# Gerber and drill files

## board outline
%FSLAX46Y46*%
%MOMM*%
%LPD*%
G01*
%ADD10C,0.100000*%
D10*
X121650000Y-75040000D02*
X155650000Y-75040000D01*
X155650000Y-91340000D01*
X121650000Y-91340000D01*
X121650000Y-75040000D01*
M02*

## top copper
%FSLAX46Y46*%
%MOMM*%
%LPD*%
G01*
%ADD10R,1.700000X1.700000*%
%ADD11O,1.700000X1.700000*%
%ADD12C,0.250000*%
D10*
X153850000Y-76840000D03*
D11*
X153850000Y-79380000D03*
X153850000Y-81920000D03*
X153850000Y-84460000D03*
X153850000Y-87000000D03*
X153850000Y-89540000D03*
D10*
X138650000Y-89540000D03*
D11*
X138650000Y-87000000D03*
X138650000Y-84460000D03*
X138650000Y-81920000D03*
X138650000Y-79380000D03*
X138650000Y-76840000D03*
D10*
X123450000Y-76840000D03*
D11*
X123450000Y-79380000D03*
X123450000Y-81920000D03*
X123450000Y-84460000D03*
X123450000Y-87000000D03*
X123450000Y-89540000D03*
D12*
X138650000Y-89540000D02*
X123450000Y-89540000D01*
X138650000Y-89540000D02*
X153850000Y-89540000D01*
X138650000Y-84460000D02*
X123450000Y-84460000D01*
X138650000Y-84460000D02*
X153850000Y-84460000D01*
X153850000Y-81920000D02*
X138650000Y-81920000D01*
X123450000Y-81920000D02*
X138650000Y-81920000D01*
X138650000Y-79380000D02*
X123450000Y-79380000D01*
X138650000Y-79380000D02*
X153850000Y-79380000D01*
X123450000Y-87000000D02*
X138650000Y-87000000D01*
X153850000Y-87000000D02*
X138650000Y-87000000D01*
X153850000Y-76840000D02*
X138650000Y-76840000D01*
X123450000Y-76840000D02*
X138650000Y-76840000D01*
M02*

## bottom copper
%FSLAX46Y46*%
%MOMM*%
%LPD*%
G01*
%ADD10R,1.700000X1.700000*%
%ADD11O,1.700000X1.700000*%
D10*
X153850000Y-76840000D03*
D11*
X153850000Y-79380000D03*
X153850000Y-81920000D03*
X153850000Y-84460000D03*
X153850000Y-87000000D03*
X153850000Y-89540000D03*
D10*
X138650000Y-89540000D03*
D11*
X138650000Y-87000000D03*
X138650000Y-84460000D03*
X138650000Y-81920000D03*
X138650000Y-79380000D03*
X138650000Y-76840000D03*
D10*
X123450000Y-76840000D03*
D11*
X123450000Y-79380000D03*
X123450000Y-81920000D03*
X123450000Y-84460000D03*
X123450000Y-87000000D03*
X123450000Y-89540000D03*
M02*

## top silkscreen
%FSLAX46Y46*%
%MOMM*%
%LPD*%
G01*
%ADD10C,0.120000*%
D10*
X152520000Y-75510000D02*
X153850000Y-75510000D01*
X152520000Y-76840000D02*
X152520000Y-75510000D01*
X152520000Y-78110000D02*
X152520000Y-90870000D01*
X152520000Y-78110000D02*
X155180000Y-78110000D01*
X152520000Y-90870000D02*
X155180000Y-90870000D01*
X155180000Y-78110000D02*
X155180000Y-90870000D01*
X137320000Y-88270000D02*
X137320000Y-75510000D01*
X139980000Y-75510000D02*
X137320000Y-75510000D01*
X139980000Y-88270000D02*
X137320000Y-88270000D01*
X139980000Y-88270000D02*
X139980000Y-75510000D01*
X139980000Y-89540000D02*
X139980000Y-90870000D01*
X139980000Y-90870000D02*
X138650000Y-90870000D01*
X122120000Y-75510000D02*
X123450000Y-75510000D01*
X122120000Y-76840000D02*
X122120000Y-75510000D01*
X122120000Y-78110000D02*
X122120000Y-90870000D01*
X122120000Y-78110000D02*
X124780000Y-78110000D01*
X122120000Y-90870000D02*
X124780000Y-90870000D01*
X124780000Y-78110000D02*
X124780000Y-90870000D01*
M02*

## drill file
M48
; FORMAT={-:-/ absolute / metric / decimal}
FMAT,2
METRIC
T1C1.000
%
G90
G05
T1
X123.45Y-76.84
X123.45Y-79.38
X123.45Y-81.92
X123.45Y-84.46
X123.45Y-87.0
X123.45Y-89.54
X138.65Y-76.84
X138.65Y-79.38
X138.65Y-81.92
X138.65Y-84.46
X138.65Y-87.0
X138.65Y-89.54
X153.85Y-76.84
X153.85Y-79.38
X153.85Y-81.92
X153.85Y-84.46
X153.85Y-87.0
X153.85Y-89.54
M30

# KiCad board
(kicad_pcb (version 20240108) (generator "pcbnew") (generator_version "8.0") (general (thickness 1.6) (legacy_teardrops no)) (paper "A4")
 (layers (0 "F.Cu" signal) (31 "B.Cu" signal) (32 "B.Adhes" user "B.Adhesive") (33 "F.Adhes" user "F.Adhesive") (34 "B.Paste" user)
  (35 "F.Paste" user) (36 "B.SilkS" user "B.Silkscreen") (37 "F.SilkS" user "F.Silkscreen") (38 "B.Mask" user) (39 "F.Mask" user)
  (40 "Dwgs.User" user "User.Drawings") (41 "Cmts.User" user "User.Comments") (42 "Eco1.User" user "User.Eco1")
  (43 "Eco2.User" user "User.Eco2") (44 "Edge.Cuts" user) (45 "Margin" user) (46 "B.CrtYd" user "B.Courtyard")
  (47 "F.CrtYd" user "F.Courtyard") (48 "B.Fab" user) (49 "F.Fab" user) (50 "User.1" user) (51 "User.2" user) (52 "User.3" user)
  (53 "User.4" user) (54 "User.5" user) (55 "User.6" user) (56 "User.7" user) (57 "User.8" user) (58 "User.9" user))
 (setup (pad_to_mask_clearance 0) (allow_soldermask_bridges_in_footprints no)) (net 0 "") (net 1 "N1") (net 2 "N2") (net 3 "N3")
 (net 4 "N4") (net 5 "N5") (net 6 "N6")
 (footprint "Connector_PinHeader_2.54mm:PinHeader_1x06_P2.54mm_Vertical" (layer "F.Cu") (at 153.85 76.84)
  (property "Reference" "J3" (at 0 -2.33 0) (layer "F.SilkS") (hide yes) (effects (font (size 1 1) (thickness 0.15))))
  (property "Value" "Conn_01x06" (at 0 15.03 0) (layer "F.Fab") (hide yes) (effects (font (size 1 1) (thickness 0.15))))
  (fp_line (start -1.33 -1.33) (end 0 -1.33) (stroke (width 0.12) (type solid)) (layer "F.SilkS"))
  (fp_line (start -1.33 0) (end -1.33 -1.33) (stroke (width 0.12) (type solid)) (layer "F.SilkS"))
  (fp_line (start -1.33 1.27) (end -1.33 14.03) (stroke (width 0.12) (type solid)) (layer "F.SilkS"))
  (fp_line (start -1.33 1.27) (end 1.33 1.27) (stroke (width 0.12) (type solid)) (layer "F.SilkS"))
  (fp_line (start -1.33 14.03) (end 1.33 14.03) (stroke (width 0.12) (type solid)) (layer "F.SilkS"))
  (fp_line (start 1.33 1.27) (end 1.33 14.03) (stroke (width 0.12) (type solid)) (layer "F.SilkS"))
  (pad "1" thru_hole rect (at 0 0) (size 1.7 1.7) (drill 1) (layers "*.Cu" "*.Mask") (remove_unused_layers no) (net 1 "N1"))
  (pad "2" thru_hole oval (at 0 2.54) (size 1.7 1.7) (drill 1) (layers "*.Cu" "*.Mask") (remove_unused_layers no) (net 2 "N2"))
  (pad "3" thru_hole oval (at 0 5.08) (size 1.7 1.7) (drill 1) (layers "*.Cu" "*.Mask") (remove_unused_layers no) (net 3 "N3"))
  (pad "4" thru_hole oval (at 0 7.62) (size 1.7 1.7) (drill 1) (layers "*.Cu" "*.Mask") (remove_unused_layers no) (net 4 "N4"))
  (pad "5" thru_hole oval (at 0 10.16) (size 1.7 1.7) (drill 1) (layers "*.Cu" "*.Mask") (remove_unused_layers no) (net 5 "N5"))
  (pad "6" thru_hole oval (at 0 12.7) (size 1.7 1.7) (drill 1) (layers "*.Cu" "*.Mask") (remove_unused_layers no) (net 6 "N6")))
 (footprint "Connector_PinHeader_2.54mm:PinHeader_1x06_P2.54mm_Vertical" (layer "F.Cu") (at 138.65 89.54 180)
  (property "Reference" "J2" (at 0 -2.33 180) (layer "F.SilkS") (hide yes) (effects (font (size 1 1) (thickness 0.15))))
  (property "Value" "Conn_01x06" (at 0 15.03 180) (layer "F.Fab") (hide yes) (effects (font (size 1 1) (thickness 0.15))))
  (fp_line (start 1.33 1.27) (end 1.33 14.03) (stroke (width 0.12) (type solid)) (layer "F.SilkS"))
  (fp_line (start -1.33 14.03) (end 1.33 14.03) (stroke (width 0.12) (type solid)) (layer "F.SilkS"))
  (fp_line (start -1.33 1.27) (end 1.33 1.27) (stroke (width 0.12) (type solid)) (layer "F.SilkS"))
  (fp_line (start -1.33 1.27) (end -1.33 14.03) (stroke (width 0.12) (type solid)) (layer "F.SilkS"))
  (fp_line (start -1.33 0) (end -1.33 -1.33) (stroke (width 0.12) (type solid)) (layer "F.SilkS"))
  (fp_line (start -1.33 -1.33) (end 0 -1.33) (stroke (width 0.12) (type solid)) (layer "F.SilkS"))
  (pad "1" thru_hole rect (at 0 0 180) (size 1.7 1.7) (drill 1) (layers "*.Cu" "*.Mask") (remove_unused_layers no) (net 6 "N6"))
  (pad "2" thru_hole oval (at 0 2.54 180) (size 1.7 1.7) (drill 1) (layers "*.Cu" "*.Mask") (remove_unused_layers no) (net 5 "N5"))
  (pad "3" thru_hole oval (at 0 5.08 180) (size 1.7 1.7) (drill 1) (layers "*.Cu" "*.Mask") (remove_unused_layers no) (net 4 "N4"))
  (pad "4" thru_hole oval (at 0 7.62 180) (size 1.7 1.7) (drill 1) (layers "*.Cu" "*.Mask") (remove_unused_layers no) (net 3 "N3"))
  (pad "5" thru_hole oval (at 0 10.16 180) (size 1.7 1.7) (drill 1) (layers "*.Cu" "*.Mask") (remove_unused_layers no) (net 2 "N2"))
  (pad "6" thru_hole oval (at 0 12.7 180) (size 1.7 1.7) (drill 1) (layers "*.Cu" "*.Mask") (remove_unused_layers no) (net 1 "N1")))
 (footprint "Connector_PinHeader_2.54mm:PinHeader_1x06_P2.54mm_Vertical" (layer "F.Cu") (at 123.45 76.84)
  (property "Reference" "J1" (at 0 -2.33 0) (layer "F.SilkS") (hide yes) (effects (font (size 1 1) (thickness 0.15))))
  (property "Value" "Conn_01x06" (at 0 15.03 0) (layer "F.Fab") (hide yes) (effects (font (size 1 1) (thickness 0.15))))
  (fp_line (start -1.33 -1.33) (end 0 -1.33) (stroke (width 0.12) (type solid)) (layer "F.SilkS"))
  (fp_line (start -1.33 0) (end -1.33 -1.33) (stroke (width 0.12) (type solid)) (layer "F.SilkS"))
  (fp_line (start -1.33 1.27) (end -1.33 14.03) (stroke (width 0.12) (type solid)) (layer "F.SilkS"))
  (fp_line (start -1.33 1.27) (end 1.33 1.27) (stroke (width 0.12) (type solid)) (layer "F.SilkS"))
  (fp_line (start -1.33 14.03) (end 1.33 14.03) (stroke (width 0.12) (type solid)) (layer "F.SilkS"))
  (fp_line (start 1.33 1.27) (end 1.33 14.03) (stroke (width 0.12) (type solid)) (layer "F.SilkS"))
  (pad "1" thru_hole rect (at 0 0) (size 1.7 1.7) (drill 1) (layers "*.Cu" "*.Mask") (remove_unused_layers no) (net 1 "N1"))
  (pad "2" thru_hole oval (at 0 2.54) (size 1.7 1.7) (drill 1) (layers "*.Cu" "*.Mask") (remove_unused_layers no) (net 2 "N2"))
  (pad "3" thru_hole oval (at 0 5.08) (size 1.7 1.7) (drill 1) (layers "*.Cu" "*.Mask") (remove_unused_layers no) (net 3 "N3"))
  (pad "4" thru_hole oval (at 0 7.62) (size 1.7 1.7) (drill 1) (layers "*.Cu" "*.Mask") (remove_unused_layers no) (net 4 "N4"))
  (pad "5" thru_hole oval (at 0 10.16) (size 1.7 1.7) (drill 1) (layers "*.Cu" "*.Mask") (remove_unused_layers no) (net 5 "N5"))
  (pad "6" thru_hole oval (at 0 12.7) (size 1.7 1.7) (drill 1) (layers "*.Cu" "*.Mask") (remove_unused_layers no) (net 6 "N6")))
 (gr_rect (start 121.65 75.04) (end 155.65 91.34) (stroke (width 0.1) (type default)) (fill none) (layer "Edge.Cuts"))
 (segment (start 138.65 89.54) (end 123.45 89.54) (width 0.25) (layer "F.Cu") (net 6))
 (segment (start 138.65 89.54) (end 153.85 89.54) (width 0.25) (layer "F.Cu") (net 6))
 (segment (start 138.65 84.46) (end 123.45 84.46) (width 0.25) (layer "F.Cu") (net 4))
 (segment (start 138.65 84.46) (end 153.85 84.46) (width 0.25) (layer "F.Cu") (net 4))
 (segment (start 153.85 81.92) (end 138.65 81.92) (width 0.25) (layer "F.Cu") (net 3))
 (segment (start 123.45 81.92) (end 138.65 81.92) (width 0.25) (layer "F.Cu") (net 3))
 (segment (start 138.65 79.38) (end 123.45 79.38) (width 0.25) (layer "F.Cu") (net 2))
 (segment (start 138.65 79.38) (end 153.85 79.38) (width 0.25) (layer "F.Cu") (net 2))
 (segment (start 123.45 87) (end 138.65 87) (width 0.25) (layer "F.Cu") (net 5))
 (segment (start 153.85 87) (end 138.65 87) (width 0.25) (layer "F.Cu") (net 5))
 (segment (start 153.85 76.84) (end 138.65 76.84) (width 0.25) (layer "F.Cu") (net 1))
 (segment (start 123.45 76.84) (end 138.65 76.84) (width 0.25) (layer "F.Cu") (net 1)))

